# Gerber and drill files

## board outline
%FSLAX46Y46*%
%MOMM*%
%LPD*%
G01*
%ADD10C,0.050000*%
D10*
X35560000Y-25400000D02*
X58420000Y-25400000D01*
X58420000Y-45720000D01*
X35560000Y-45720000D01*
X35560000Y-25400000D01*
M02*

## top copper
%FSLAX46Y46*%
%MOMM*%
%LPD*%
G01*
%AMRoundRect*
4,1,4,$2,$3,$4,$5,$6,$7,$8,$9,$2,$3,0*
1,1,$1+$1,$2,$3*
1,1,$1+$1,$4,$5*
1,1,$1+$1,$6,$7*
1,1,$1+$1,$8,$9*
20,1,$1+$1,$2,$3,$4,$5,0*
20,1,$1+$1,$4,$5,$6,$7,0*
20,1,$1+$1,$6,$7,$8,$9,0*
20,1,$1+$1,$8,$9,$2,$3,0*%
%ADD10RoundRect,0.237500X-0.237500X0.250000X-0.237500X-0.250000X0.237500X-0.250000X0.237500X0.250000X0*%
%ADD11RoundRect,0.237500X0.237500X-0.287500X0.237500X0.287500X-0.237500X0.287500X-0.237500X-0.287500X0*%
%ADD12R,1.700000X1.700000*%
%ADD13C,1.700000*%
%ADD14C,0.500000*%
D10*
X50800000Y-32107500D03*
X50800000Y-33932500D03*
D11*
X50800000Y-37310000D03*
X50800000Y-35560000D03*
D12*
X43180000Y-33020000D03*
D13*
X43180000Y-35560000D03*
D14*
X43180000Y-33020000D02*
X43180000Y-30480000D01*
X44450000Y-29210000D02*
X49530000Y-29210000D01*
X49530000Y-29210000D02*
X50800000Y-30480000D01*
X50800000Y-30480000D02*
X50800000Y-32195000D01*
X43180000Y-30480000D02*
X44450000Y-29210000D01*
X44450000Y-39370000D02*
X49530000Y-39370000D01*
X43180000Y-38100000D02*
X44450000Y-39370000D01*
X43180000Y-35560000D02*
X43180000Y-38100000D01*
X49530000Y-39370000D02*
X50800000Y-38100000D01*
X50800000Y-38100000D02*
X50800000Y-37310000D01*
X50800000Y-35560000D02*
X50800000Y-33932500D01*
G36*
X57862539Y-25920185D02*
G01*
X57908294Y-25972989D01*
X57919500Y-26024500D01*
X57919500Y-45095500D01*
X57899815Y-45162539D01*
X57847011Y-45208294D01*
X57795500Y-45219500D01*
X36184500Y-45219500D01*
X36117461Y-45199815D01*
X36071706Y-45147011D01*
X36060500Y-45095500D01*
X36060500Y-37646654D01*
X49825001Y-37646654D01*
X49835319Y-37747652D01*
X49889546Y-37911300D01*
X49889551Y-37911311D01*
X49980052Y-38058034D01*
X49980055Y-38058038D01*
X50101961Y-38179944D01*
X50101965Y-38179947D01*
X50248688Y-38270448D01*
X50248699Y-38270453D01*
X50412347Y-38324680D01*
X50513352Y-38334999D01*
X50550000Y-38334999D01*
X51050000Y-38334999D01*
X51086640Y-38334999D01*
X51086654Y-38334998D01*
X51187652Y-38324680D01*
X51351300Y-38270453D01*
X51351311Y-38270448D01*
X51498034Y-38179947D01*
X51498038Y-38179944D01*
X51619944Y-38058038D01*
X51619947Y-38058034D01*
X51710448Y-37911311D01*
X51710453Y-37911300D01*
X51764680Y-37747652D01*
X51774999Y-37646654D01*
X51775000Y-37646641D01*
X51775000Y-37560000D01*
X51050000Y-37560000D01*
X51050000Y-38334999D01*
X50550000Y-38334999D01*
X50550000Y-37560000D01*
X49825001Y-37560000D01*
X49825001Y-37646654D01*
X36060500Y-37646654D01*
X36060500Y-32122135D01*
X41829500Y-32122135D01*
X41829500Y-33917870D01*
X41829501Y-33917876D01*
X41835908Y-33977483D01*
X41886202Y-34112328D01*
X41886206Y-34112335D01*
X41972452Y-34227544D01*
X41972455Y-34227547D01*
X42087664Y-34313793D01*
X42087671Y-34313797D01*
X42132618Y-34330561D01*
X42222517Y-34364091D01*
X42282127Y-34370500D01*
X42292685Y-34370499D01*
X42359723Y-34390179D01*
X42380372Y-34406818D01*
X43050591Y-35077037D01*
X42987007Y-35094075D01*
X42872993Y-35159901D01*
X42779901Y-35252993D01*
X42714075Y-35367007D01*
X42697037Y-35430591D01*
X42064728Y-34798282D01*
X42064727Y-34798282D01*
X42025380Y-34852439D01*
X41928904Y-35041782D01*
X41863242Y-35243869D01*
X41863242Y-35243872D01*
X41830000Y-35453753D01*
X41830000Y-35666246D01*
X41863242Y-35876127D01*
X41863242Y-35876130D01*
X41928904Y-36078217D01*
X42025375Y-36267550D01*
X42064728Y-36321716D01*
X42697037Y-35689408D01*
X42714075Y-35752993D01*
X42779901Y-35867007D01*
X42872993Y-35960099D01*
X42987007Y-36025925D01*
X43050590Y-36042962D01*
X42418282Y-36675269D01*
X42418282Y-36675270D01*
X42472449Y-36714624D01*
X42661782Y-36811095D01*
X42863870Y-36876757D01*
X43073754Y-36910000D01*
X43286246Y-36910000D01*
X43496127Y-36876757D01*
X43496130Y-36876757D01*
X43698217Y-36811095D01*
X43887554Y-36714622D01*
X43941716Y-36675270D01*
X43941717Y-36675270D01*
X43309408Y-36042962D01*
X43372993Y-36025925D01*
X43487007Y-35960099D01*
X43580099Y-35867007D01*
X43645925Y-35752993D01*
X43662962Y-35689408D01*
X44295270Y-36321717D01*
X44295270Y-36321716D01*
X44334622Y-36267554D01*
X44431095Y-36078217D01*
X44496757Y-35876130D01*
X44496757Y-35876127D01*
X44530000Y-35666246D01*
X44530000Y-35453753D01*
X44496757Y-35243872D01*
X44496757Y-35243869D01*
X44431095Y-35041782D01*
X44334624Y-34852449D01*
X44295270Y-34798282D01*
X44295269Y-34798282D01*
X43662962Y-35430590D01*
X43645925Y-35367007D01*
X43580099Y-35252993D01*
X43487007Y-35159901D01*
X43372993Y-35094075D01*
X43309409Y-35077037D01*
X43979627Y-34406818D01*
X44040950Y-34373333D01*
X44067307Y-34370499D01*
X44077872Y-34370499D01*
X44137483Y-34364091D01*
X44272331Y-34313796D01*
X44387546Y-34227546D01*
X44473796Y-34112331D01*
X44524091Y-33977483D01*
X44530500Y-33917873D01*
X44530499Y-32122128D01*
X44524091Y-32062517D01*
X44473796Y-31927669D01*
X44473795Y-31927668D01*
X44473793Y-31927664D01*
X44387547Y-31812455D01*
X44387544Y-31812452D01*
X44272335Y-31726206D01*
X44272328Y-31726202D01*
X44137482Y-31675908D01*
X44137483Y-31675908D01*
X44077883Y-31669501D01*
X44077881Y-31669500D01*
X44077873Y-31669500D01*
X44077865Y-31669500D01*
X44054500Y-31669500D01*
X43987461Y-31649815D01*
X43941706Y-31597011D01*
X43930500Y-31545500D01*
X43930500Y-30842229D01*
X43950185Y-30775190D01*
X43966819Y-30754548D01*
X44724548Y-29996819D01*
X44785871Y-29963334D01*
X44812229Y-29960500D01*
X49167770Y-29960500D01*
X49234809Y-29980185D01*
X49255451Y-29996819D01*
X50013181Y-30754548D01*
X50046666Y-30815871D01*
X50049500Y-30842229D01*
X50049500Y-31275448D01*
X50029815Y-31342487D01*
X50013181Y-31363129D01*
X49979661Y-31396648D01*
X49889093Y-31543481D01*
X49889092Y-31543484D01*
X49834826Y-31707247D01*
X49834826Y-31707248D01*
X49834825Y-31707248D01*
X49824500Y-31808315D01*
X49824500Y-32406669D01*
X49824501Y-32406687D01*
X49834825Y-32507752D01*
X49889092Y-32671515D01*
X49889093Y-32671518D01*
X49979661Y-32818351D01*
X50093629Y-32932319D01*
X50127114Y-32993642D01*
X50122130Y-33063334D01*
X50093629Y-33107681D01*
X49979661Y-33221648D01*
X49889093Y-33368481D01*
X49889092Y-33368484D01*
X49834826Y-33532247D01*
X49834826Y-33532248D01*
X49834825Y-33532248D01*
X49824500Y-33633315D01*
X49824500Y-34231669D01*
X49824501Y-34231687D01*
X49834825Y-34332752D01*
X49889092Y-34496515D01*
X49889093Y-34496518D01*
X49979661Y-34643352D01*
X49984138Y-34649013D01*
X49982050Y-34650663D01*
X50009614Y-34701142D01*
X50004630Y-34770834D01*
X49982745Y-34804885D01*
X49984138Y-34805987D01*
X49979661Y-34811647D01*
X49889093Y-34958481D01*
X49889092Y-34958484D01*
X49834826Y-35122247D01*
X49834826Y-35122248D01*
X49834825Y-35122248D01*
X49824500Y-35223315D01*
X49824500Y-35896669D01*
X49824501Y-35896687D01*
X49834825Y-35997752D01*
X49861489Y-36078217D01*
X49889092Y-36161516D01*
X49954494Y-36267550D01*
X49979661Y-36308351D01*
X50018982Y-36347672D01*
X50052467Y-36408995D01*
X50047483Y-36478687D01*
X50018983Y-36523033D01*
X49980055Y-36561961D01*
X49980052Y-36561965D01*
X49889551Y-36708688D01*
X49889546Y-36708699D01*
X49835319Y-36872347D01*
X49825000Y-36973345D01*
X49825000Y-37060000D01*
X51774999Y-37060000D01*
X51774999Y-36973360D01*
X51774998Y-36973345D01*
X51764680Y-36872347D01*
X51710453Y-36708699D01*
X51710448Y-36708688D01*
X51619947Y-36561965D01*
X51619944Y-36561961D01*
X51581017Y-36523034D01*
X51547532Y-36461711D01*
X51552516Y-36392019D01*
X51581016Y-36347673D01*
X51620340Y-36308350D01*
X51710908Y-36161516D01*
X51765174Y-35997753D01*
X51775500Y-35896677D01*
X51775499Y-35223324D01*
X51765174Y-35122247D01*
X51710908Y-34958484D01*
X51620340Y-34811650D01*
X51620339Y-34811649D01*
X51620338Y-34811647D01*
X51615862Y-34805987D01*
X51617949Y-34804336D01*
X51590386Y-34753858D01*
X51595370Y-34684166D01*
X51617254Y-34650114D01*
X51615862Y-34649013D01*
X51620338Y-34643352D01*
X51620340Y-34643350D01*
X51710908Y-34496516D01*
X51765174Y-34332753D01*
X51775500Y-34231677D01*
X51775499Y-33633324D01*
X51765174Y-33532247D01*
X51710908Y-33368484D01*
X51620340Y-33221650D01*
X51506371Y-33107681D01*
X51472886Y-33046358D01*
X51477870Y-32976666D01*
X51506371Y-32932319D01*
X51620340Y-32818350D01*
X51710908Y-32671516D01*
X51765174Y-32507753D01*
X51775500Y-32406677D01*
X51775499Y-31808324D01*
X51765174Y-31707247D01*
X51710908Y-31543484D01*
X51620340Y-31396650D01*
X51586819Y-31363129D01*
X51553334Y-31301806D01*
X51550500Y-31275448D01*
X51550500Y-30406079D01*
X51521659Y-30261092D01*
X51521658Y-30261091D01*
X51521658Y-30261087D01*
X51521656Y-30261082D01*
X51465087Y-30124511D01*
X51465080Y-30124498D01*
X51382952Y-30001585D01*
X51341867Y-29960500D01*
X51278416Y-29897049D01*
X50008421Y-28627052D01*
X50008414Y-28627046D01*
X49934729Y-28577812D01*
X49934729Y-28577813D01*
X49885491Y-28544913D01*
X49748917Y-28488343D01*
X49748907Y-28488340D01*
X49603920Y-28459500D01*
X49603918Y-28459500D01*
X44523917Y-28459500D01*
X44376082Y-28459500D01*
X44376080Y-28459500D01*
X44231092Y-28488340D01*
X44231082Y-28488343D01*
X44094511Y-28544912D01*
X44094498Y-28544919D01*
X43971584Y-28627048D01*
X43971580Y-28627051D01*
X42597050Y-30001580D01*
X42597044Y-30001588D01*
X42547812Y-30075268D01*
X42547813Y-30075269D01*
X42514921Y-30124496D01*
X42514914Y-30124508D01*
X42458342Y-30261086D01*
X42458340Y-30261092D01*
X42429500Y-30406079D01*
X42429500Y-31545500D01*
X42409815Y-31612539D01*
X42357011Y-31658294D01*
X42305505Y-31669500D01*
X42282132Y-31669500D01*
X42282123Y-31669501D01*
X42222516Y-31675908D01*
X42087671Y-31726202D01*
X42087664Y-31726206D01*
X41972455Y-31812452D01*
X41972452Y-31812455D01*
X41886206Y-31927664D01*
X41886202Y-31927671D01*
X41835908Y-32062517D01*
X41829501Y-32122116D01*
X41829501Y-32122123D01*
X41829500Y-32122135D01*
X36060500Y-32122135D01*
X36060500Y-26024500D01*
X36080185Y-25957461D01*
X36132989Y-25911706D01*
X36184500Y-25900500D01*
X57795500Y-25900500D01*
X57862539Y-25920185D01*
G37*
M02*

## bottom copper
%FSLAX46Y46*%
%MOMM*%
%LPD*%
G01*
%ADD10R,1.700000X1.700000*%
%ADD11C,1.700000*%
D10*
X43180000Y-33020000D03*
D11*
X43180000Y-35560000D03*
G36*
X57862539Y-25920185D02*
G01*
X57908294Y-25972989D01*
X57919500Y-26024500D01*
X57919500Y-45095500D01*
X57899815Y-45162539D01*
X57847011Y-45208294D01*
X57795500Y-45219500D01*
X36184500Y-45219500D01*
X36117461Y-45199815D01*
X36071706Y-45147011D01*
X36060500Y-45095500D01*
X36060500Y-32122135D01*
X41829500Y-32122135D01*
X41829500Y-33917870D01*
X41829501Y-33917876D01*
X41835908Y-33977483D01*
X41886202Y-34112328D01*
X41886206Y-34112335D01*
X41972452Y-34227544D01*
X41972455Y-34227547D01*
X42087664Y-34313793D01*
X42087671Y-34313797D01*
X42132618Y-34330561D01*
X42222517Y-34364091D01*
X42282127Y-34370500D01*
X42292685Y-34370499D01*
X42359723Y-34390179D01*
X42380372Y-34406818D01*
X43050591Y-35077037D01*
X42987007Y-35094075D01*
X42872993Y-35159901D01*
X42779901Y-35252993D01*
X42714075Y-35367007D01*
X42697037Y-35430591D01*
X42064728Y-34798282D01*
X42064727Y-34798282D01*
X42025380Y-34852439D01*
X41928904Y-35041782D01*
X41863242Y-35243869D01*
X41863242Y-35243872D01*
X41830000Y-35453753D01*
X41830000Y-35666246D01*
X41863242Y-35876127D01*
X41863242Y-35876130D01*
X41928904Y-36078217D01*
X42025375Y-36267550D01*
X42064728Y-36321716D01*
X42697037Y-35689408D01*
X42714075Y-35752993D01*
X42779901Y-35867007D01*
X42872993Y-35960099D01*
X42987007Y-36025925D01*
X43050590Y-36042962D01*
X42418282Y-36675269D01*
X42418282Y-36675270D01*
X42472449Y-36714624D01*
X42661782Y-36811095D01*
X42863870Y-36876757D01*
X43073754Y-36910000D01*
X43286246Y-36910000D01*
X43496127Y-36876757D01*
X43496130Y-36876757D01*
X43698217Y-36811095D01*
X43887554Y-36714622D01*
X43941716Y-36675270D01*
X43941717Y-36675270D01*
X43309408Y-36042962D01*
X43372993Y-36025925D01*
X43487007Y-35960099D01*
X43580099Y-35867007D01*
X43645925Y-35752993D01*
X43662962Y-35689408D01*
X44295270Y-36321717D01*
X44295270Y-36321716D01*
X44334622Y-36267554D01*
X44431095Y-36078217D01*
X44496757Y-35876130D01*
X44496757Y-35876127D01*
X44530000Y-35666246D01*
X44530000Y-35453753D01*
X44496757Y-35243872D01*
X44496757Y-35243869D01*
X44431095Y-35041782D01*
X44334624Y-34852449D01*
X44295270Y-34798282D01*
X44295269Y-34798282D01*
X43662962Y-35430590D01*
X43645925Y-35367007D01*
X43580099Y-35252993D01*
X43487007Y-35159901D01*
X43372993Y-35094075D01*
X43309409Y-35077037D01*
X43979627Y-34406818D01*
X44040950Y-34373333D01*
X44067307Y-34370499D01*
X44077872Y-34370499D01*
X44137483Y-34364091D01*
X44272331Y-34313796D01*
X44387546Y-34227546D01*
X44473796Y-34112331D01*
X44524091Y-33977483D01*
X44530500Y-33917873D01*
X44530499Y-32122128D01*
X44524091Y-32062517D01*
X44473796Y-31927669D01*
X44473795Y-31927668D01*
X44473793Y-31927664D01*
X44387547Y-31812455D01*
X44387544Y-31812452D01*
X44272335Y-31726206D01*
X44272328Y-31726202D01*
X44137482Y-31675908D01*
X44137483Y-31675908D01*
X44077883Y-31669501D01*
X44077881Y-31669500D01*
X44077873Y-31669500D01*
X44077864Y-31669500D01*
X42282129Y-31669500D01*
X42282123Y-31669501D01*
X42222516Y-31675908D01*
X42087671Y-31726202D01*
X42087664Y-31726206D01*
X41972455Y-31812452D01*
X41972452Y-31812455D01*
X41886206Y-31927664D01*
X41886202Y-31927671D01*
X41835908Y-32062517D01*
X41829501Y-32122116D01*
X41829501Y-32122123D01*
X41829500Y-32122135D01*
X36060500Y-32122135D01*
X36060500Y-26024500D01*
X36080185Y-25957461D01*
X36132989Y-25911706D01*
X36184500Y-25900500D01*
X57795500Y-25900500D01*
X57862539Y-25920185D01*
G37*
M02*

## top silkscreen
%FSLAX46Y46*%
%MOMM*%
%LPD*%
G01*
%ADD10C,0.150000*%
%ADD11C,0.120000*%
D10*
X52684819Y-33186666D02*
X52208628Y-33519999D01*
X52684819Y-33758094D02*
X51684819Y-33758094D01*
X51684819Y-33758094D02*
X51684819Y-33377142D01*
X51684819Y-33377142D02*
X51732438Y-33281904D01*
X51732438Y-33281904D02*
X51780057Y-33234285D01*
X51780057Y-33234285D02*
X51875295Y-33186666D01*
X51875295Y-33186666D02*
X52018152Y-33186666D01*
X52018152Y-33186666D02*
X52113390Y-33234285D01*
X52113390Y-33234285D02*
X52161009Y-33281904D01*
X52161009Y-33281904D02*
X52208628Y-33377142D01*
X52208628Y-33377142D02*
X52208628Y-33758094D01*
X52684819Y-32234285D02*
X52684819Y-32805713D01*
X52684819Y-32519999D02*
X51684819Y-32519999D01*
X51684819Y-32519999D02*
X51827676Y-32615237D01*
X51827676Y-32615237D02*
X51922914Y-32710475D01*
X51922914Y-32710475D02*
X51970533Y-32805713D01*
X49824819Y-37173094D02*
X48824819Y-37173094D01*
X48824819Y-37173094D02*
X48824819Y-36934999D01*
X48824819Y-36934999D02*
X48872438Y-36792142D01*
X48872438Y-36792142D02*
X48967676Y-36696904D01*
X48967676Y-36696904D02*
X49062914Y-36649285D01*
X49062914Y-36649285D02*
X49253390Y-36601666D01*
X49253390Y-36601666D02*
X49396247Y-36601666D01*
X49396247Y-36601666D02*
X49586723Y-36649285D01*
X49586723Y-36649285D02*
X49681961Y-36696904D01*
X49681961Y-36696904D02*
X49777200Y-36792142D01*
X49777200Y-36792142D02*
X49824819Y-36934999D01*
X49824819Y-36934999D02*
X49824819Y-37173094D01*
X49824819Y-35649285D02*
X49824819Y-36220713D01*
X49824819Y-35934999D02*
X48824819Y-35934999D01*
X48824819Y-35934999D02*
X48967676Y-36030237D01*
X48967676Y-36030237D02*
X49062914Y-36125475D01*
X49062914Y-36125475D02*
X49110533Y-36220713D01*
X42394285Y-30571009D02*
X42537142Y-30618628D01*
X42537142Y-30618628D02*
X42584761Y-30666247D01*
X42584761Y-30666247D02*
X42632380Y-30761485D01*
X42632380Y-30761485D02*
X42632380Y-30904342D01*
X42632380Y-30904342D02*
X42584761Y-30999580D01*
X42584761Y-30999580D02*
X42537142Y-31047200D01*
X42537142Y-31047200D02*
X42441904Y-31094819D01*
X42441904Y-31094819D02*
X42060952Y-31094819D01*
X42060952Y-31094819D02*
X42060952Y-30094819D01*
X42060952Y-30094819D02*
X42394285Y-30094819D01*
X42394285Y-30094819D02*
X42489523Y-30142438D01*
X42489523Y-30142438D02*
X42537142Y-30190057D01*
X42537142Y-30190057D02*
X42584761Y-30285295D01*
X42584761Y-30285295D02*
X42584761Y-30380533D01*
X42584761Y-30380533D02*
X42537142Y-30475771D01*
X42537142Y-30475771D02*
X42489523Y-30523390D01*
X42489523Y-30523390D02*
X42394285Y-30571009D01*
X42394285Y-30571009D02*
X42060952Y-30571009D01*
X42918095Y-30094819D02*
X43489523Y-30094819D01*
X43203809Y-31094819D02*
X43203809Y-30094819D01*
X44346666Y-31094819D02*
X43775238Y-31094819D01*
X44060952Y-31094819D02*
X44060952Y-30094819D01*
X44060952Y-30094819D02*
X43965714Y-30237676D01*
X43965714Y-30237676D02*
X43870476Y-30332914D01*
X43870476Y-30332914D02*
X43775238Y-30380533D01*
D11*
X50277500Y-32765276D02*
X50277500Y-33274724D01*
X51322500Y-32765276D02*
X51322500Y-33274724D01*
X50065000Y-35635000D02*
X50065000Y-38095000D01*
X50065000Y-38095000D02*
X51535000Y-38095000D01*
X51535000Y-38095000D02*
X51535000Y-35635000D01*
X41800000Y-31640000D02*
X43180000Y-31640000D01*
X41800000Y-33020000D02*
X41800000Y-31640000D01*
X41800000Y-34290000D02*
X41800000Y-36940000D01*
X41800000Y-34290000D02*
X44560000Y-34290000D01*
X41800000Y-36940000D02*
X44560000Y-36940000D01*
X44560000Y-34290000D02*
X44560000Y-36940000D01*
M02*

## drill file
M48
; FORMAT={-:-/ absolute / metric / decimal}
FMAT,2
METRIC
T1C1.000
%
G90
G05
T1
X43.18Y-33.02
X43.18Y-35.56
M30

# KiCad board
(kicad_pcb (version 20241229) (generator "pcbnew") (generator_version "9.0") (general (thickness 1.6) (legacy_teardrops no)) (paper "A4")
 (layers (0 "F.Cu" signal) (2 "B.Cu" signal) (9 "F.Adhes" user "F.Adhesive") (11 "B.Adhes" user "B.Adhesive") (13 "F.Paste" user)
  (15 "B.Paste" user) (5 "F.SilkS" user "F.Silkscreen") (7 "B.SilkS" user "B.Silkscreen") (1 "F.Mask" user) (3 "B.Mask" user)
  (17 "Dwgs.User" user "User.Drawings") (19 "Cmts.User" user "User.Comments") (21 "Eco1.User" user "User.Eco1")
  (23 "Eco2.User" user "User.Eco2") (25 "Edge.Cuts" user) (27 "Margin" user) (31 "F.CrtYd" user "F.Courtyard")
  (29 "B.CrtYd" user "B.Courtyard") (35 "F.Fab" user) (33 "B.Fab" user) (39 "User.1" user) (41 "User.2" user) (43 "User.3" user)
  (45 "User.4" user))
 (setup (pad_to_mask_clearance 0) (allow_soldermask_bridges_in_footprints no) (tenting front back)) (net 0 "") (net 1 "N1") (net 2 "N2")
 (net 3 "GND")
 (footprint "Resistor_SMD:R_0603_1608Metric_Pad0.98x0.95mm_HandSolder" (layer "F.Cu") (at 50.8 33.02 -90)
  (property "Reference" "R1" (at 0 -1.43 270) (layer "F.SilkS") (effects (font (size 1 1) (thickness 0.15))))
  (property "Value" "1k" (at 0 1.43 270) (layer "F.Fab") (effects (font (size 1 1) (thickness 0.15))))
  (fp_line (start -0.254724 0.5225) (end 0.254724 0.5225) (stroke (width 0.12) (type solid)) (layer "F.SilkS"))
  (fp_line (start -0.254724 -0.5225) (end 0.254724 -0.5225) (stroke (width 0.12) (type solid)) (layer "F.SilkS"))
  (pad "1" smd roundrect (at -0.9125 0 270) (size 0.975 0.95) (layers "F.Cu" "F.Mask" "F.Paste") (roundrect_rratio 0.25) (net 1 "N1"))
  (pad "2" smd roundrect (at 0.9125 0 270) (size 0.975 0.95) (layers "F.Cu" "F.Mask" "F.Paste") (roundrect_rratio 0.25) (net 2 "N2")))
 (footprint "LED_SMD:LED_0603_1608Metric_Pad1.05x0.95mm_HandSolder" (layer "F.Cu") (at 50.8 36.435 90)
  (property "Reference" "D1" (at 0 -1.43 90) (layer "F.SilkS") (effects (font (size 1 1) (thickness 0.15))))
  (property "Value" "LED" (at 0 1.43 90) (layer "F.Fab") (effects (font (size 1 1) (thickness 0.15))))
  (fp_line (start 0.8 -0.735) (end -1.66 -0.735) (stroke (width 0.12) (type solid)) (layer "F.SilkS"))
  (fp_line (start -1.66 -0.735) (end -1.66 0.735) (stroke (width 0.12) (type solid)) (layer "F.SilkS"))
  (fp_line (start -1.66 0.735) (end 0.8 0.735) (stroke (width 0.12) (type solid)) (layer "F.SilkS"))
  (pad "1" smd roundrect (at -0.875 0 90) (size 1.05 0.95) (layers "F.Cu" "F.Mask" "F.Paste") (roundrect_rratio 0.25) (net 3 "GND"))
  (pad "2" smd roundrect (at 0.875 0 90) (size 1.05 0.95) (layers "F.Cu" "F.Mask" "F.Paste") (roundrect_rratio 0.25) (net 2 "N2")))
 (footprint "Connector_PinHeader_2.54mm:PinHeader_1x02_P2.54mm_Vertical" (layer "F.Cu") (at 43.18 33.02)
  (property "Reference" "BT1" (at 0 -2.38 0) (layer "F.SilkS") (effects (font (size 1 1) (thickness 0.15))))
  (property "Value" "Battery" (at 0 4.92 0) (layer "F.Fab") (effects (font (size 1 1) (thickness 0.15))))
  (fp_line (start -1.38 -1.38) (end 0 -1.38) (stroke (width 0.12) (type solid)) (layer "F.SilkS"))
  (fp_line (start -1.38 0) (end -1.38 -1.38) (stroke (width 0.12) (type solid)) (layer "F.SilkS"))
  (fp_line (start -1.38 1.27) (end -1.38 3.92) (stroke (width 0.12) (type solid)) (layer "F.SilkS"))
  (fp_line (start -1.38 1.27) (end 1.38 1.27) (stroke (width 0.12) (type solid)) (layer "F.SilkS"))
  (fp_line (start -1.38 3.92) (end 1.38 3.92) (stroke (width 0.12) (type solid)) (layer "F.SilkS"))
  (fp_line (start 1.38 1.27) (end 1.38 3.92) (stroke (width 0.12) (type solid)) (layer "F.SilkS"))
  (pad "1" thru_hole rect (at 0 0) (size 1.7 1.7) (drill 1) (layers "*.Cu" "*.Mask") (remove_unused_layers no) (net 1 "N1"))
  (pad "2" thru_hole circle (at 0 2.54) (size 1.7 1.7) (drill 1) (layers "*.Cu" "*.Mask") (remove_unused_layers no) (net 3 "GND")))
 (gr_rect (start 35.56 25.4) (end 58.42 45.72) (stroke (width 0.05) (type default)) (fill no) (layer "Edge.Cuts"))
 (segment (start 43.18 33.02) (end 43.18 30.48) (width 0.5) (layer "F.Cu") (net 1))
 (segment (start 44.45 29.21) (end 49.53 29.21) (width 0.5) (layer "F.Cu") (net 1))
 (segment (start 49.53 29.21) (end 50.8 30.48) (width 0.5) (layer "F.Cu") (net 1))
 (segment (start 50.8 30.48) (end 50.8 32.195) (width 0.5) (layer "F.Cu") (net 1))
 (segment (start 43.18 30.48) (end 44.45 29.21) (width 0.5) (layer "F.Cu") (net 1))
 (segment (start 44.45 39.37) (end 49.53 39.37) (width 0.5) (layer "F.Cu") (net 3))
 (segment (start 43.18 38.1) (end 44.45 39.37) (width 0.5) (layer "F.Cu") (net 3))
 (segment (start 43.18 35.56) (end 43.18 38.1) (width 0.5) (layer "F.Cu") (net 3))
 (segment (start 49.53 39.37) (end 50.8 38.1) (width 0.5) (layer "F.Cu") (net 3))
 (segment (start 50.8 38.1) (end 50.8 37.31) (width 0.5) (layer "F.Cu") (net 3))
 (segment (start 50.8 35.56) (end 50.8 33.9325) (width 0.5) (layer "F.Cu") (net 2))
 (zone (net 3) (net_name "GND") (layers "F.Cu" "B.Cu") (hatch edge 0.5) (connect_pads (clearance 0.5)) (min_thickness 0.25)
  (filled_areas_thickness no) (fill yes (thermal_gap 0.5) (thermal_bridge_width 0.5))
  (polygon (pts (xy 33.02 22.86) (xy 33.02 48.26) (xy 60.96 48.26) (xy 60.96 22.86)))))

